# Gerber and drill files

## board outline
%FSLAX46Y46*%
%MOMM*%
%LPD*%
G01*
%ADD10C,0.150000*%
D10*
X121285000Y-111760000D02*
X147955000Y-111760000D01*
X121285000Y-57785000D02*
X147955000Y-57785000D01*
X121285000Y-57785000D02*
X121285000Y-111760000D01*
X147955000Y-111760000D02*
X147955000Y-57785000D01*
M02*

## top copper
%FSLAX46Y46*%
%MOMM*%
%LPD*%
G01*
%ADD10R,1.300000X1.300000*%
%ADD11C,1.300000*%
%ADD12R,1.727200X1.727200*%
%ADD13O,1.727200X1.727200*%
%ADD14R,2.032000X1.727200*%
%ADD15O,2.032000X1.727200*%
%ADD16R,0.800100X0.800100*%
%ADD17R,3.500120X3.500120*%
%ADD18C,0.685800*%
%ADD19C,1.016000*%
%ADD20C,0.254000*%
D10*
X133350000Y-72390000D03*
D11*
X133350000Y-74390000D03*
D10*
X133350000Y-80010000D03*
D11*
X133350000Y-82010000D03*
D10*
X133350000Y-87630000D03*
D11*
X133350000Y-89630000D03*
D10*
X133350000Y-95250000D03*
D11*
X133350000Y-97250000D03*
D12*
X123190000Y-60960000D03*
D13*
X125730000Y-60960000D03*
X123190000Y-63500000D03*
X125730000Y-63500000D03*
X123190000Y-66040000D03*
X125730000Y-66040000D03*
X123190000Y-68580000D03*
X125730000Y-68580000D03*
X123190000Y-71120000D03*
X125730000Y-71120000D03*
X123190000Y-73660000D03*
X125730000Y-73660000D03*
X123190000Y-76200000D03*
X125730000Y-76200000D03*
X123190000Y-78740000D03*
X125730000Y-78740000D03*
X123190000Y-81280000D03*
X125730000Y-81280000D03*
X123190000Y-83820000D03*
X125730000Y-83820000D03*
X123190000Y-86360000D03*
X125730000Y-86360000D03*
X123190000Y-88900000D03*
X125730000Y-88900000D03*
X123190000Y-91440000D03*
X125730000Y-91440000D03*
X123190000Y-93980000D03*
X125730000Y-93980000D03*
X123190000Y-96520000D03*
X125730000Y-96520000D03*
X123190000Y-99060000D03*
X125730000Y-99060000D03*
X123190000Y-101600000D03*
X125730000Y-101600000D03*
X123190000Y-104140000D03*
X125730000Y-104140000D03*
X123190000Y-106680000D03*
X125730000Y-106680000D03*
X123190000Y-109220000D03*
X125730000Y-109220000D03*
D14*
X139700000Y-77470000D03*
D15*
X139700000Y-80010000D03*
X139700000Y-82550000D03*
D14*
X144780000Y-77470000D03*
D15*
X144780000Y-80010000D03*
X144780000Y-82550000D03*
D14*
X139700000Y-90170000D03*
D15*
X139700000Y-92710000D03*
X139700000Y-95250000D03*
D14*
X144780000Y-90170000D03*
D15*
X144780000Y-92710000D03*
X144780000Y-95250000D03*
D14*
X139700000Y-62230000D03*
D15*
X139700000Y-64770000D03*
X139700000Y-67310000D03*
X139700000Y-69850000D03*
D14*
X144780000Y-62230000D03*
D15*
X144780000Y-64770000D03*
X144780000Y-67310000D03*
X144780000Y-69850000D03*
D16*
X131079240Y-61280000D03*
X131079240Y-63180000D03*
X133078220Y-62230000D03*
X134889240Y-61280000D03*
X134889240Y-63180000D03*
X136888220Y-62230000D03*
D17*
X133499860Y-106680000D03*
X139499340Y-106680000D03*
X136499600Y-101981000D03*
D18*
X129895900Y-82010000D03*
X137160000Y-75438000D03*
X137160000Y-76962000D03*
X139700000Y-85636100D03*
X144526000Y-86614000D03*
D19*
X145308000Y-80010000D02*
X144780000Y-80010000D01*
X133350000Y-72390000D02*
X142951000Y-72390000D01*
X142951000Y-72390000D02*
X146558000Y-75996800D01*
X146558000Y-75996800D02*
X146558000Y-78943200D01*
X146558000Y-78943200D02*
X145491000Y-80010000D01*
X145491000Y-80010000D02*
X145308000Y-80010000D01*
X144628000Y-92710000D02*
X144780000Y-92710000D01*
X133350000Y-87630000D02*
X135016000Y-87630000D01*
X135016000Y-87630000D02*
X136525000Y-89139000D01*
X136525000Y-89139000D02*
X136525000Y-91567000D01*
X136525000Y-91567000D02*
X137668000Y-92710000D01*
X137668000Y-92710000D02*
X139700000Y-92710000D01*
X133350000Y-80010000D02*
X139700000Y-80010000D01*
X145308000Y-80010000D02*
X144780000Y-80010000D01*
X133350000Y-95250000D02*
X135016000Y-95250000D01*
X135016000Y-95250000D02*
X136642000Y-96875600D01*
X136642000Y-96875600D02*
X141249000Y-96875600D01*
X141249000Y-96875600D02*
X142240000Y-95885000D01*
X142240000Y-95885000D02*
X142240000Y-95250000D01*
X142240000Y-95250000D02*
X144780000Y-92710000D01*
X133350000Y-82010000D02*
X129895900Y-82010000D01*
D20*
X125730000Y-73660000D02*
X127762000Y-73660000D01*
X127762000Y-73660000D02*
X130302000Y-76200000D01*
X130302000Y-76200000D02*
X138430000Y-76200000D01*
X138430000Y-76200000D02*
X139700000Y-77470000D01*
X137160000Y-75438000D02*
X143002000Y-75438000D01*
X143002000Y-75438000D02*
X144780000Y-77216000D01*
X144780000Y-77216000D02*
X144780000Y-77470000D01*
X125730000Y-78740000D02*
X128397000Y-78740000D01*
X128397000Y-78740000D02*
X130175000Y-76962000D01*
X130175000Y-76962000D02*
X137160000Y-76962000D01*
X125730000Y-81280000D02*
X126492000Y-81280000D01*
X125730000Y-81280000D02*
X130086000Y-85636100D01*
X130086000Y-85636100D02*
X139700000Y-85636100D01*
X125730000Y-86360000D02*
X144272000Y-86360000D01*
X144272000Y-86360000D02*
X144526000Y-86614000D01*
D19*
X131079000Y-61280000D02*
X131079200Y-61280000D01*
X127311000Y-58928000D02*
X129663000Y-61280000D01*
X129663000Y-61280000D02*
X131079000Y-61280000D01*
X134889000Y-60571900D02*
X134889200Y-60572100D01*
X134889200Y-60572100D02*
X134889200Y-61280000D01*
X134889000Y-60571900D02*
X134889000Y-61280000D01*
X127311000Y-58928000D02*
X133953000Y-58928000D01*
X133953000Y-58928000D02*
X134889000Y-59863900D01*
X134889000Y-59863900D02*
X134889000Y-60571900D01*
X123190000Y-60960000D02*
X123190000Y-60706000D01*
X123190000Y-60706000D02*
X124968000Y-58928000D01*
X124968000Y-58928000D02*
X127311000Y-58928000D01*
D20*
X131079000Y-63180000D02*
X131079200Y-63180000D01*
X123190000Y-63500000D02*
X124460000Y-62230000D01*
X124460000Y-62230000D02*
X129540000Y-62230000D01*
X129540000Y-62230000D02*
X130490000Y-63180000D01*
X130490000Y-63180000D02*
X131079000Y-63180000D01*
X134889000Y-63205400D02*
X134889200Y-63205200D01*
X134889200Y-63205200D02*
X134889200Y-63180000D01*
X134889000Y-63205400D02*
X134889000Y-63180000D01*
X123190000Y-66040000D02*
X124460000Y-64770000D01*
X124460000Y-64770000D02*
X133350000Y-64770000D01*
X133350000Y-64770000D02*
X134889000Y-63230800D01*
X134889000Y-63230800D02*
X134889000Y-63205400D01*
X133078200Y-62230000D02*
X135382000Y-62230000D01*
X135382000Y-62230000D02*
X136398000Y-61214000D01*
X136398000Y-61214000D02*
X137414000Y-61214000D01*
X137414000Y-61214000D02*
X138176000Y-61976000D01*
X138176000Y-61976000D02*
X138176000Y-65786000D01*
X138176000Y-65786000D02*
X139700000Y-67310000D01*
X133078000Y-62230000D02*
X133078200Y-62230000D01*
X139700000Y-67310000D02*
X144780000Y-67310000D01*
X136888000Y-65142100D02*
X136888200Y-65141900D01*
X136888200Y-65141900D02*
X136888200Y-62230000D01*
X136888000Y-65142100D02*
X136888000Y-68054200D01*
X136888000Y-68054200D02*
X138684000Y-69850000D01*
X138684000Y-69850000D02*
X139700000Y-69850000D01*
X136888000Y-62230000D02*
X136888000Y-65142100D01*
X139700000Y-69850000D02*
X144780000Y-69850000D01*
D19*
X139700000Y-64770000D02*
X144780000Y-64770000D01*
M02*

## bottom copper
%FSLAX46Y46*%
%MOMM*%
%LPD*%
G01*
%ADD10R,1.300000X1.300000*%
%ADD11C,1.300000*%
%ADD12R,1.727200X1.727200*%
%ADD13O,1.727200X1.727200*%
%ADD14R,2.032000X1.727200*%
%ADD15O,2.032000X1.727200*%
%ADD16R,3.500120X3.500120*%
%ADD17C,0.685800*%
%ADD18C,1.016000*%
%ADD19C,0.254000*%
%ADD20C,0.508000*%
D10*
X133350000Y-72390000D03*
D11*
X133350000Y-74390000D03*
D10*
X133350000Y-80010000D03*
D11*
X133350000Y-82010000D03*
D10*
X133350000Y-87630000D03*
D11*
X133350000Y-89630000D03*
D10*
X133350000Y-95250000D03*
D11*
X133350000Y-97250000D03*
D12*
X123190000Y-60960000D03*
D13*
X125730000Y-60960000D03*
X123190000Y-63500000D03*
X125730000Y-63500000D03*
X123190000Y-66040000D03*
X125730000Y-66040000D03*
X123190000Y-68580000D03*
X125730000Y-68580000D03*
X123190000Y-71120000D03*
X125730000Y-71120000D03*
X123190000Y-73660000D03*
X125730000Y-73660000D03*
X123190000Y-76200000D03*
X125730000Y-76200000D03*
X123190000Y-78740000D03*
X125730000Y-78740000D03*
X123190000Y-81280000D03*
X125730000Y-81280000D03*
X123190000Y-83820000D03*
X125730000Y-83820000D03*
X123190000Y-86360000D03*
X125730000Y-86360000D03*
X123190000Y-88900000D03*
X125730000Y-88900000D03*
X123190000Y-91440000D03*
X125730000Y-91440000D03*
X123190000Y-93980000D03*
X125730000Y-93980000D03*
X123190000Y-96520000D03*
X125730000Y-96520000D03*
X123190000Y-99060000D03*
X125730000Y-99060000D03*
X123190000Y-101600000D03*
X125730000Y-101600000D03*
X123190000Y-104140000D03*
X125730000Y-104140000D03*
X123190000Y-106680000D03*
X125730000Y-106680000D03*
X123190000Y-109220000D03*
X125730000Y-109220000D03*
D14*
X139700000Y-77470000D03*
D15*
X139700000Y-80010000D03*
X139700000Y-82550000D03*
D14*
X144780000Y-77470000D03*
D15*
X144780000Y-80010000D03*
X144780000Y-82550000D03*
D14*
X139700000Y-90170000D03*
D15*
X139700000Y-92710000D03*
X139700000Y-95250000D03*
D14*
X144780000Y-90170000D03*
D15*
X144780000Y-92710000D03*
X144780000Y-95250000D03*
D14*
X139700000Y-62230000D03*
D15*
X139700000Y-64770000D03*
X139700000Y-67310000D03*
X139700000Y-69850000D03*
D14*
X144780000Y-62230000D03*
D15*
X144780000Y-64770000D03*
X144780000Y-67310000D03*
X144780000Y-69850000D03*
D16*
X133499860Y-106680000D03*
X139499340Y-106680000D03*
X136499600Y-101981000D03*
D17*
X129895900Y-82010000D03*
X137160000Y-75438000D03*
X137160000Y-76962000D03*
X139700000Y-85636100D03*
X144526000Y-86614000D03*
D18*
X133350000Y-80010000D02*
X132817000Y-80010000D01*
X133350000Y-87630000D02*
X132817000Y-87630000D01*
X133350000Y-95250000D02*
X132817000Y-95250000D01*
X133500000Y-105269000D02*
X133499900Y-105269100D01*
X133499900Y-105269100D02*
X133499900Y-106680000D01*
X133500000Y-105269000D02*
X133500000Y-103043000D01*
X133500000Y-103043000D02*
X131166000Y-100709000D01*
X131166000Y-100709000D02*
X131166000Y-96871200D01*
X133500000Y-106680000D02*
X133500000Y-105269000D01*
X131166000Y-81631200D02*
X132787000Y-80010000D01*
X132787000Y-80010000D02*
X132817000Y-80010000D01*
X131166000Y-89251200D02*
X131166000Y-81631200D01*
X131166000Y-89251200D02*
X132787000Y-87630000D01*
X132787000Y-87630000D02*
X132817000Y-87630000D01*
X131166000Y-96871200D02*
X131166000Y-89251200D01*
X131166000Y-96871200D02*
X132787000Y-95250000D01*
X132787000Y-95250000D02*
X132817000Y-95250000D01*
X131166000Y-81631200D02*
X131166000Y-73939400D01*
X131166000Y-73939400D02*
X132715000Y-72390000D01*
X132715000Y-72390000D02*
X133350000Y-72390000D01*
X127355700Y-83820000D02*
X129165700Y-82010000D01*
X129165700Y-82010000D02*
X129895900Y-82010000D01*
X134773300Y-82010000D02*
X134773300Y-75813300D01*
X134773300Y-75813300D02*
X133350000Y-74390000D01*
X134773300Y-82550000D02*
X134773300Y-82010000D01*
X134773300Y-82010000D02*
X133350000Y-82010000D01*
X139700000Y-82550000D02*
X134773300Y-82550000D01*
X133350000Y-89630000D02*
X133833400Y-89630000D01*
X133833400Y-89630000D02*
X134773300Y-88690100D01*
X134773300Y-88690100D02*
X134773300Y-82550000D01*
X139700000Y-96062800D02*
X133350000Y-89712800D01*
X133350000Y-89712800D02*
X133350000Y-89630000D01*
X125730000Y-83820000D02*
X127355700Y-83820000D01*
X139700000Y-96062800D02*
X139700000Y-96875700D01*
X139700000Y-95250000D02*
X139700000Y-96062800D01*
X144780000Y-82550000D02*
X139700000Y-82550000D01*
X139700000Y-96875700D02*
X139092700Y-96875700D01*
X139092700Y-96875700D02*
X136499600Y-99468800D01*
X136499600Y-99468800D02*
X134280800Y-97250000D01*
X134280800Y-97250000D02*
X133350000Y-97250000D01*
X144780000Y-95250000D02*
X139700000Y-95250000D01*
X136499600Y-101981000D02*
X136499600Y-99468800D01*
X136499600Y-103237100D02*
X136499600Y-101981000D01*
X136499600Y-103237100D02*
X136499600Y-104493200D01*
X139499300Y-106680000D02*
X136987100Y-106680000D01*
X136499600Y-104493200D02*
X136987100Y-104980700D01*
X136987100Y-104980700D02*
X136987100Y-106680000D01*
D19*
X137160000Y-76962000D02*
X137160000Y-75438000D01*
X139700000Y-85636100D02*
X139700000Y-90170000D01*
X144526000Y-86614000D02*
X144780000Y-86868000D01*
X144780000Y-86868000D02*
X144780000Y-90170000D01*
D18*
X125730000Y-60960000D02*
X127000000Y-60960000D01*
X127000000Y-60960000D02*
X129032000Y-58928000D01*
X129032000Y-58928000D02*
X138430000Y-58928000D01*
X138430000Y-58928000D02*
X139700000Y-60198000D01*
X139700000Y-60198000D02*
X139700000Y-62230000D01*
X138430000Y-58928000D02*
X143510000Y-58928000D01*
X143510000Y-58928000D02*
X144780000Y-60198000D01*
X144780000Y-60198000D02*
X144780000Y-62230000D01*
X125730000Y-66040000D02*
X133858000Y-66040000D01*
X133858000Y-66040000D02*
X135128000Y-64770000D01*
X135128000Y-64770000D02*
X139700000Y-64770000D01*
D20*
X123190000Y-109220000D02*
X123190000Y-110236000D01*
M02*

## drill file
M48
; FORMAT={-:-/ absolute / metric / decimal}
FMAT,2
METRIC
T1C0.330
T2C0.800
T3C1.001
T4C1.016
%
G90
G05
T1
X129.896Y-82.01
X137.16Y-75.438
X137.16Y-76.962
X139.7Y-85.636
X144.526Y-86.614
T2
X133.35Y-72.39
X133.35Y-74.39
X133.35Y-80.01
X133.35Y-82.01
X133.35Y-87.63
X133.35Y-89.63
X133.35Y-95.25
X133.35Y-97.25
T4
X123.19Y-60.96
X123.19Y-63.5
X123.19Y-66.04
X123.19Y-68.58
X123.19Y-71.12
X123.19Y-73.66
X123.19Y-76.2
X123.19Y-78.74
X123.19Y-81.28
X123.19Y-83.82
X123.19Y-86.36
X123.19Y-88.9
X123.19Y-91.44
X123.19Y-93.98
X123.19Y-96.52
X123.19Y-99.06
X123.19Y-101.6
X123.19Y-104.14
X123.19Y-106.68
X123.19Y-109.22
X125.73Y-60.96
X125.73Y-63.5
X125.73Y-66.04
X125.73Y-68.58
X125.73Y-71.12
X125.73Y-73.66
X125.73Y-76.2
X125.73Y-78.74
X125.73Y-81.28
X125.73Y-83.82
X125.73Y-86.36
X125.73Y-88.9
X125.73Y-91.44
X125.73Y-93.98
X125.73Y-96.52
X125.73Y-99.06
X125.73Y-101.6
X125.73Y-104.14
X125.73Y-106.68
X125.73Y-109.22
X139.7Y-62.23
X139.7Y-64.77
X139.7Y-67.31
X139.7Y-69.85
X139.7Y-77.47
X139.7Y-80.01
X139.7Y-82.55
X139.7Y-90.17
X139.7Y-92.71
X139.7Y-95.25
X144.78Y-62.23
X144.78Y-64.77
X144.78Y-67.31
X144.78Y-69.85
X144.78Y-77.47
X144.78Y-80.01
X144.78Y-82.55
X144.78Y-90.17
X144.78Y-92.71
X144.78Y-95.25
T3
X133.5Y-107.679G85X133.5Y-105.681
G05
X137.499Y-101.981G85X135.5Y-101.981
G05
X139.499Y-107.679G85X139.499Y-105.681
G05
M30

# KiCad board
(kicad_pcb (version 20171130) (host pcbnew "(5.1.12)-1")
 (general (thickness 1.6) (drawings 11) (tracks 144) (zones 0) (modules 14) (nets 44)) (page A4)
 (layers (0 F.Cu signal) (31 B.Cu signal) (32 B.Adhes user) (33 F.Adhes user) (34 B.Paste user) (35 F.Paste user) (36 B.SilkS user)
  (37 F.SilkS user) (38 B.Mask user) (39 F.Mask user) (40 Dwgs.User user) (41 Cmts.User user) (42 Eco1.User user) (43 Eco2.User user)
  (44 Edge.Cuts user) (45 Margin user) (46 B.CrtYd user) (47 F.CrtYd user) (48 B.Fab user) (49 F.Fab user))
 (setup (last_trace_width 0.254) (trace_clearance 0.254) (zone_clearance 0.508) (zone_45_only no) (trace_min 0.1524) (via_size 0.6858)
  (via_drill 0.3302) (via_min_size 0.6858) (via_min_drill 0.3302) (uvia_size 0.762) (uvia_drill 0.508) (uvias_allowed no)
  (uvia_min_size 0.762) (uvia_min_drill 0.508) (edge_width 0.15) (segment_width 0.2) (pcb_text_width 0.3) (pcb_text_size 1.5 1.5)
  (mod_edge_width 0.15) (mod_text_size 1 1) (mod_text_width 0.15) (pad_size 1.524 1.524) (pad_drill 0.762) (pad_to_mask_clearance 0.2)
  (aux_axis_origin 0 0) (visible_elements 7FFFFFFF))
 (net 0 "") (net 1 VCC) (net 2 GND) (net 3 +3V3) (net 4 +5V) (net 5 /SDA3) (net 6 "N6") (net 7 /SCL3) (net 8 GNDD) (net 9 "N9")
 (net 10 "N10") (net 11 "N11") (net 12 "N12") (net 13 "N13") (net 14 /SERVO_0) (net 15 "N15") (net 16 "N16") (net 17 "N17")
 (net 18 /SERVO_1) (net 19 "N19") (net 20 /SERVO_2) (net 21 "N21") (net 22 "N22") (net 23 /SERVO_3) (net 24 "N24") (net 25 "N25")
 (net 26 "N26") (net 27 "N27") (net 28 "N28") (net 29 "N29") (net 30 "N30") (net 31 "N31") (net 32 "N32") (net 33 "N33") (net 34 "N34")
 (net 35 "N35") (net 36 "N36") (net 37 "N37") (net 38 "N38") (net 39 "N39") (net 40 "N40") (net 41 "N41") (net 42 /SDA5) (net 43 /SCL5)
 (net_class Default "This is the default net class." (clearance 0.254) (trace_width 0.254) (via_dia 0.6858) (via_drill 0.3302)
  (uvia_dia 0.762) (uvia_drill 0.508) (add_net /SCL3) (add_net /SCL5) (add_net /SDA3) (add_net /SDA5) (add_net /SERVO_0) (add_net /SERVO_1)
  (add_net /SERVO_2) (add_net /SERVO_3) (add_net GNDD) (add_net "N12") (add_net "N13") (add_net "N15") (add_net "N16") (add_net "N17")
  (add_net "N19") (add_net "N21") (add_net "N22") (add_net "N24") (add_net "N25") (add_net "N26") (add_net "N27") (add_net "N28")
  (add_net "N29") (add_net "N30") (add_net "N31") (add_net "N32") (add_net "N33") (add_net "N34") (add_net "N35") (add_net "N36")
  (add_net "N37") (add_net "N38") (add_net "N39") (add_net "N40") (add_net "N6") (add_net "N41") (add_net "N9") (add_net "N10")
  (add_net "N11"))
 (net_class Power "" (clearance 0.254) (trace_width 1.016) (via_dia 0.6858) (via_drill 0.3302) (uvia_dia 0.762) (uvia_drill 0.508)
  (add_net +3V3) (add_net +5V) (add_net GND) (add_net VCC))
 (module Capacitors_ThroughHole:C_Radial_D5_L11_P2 (layer F.Cu) (at 133.35 72.39 270)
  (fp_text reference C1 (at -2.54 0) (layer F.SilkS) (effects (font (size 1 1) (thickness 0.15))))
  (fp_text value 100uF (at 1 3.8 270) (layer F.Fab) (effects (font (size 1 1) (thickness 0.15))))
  (pad 1 thru_hole rect (at 0 0 270) (size 1.3 1.3) (drill 0.8) (layers *.Cu *.Mask F.SilkS) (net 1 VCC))
  (pad 2 thru_hole circle (at 2 0 270) (size 1.3 1.3) (drill 0.8) (layers *.Cu *.Mask F.SilkS) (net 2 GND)))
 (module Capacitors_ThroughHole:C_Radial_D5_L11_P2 (layer F.Cu) (at 133.35 80.01 270)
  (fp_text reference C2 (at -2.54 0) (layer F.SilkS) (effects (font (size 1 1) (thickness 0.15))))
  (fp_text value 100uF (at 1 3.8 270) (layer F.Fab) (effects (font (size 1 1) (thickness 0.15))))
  (pad 1 thru_hole rect (at 0 0 270) (size 1.3 1.3) (drill 0.8) (layers *.Cu *.Mask F.SilkS) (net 1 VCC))
  (pad 2 thru_hole circle (at 2 0 270) (size 1.3 1.3) (drill 0.8) (layers *.Cu *.Mask F.SilkS) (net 2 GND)))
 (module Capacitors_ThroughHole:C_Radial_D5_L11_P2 (layer F.Cu) (at 133.35 87.63 270)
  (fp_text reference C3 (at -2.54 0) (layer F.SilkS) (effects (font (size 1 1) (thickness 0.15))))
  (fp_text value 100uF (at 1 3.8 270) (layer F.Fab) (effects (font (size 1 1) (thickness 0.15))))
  (pad 1 thru_hole rect (at 0 0 270) (size 1.3 1.3) (drill 0.8) (layers *.Cu *.Mask F.SilkS) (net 1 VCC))
  (pad 2 thru_hole circle (at 2 0 270) (size 1.3 1.3) (drill 0.8) (layers *.Cu *.Mask F.SilkS) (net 2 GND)))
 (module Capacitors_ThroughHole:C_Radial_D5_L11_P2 (layer F.Cu) (at 133.35 95.25 270)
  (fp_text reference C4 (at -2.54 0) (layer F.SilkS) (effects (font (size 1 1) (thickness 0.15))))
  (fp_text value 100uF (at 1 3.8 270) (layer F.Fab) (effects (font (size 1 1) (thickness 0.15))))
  (pad 1 thru_hole rect (at 0 0 270) (size 1.3 1.3) (drill 0.8) (layers *.Cu *.Mask F.SilkS) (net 1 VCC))
  (pad 2 thru_hole circle (at 2 0 270) (size 1.3 1.3) (drill 0.8) (layers *.Cu *.Mask F.SilkS) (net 2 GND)))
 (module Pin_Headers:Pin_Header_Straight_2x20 (layer F.Cu) (at 123.19 60.96)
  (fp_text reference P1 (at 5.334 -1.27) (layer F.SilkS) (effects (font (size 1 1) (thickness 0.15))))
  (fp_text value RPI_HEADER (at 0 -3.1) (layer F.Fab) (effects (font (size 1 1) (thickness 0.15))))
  (pad 1 thru_hole rect (at 0 0) (size 1.7272 1.7272) (drill 1.016) (layers *.Cu *.Mask F.SilkS) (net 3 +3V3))
  (pad 2 thru_hole oval (at 2.54 0) (size 1.7272 1.7272) (drill 1.016) (layers *.Cu *.Mask F.SilkS) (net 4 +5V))
  (pad 3 thru_hole oval (at 0 2.54) (size 1.7272 1.7272) (drill 1.016) (layers *.Cu *.Mask F.SilkS) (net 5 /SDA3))
  (pad 4 thru_hole oval (at 2.54 2.54) (size 1.7272 1.7272) (drill 1.016) (layers *.Cu *.Mask F.SilkS) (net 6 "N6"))
  (pad 5 thru_hole oval (at 0 5.08) (size 1.7272 1.7272) (drill 1.016) (layers *.Cu *.Mask F.SilkS) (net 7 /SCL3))
  (pad 6 thru_hole oval (at 2.54 5.08) (size 1.7272 1.7272) (drill 1.016) (layers *.Cu *.Mask F.SilkS) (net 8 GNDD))
  (pad 7 thru_hole oval (at 0 7.62) (size 1.7272 1.7272) (drill 1.016) (layers *.Cu *.Mask F.SilkS) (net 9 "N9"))
  (pad 8 thru_hole oval (at 2.54 7.62) (size 1.7272 1.7272) (drill 1.016) (layers *.Cu *.Mask F.SilkS) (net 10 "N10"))
  (pad 9 thru_hole oval (at 0 10.16) (size 1.7272 1.7272) (drill 1.016) (layers *.Cu *.Mask F.SilkS) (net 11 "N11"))
  (pad 10 thru_hole oval (at 2.54 10.16) (size 1.7272 1.7272) (drill 1.016) (layers *.Cu *.Mask F.SilkS) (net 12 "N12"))
  (pad 11 thru_hole oval (at 0 12.7) (size 1.7272 1.7272) (drill 1.016) (layers *.Cu *.Mask F.SilkS) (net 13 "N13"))
  (pad 12 thru_hole oval (at 2.54 12.7) (size 1.7272 1.7272) (drill 1.016) (layers *.Cu *.Mask F.SilkS) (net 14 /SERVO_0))
  (pad 13 thru_hole oval (at 0 15.24) (size 1.7272 1.7272) (drill 1.016) (layers *.Cu *.Mask F.SilkS) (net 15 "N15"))
  (pad 14 thru_hole oval (at 2.54 15.24) (size 1.7272 1.7272) (drill 1.016) (layers *.Cu *.Mask F.SilkS) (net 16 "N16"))
  (pad 15 thru_hole oval (at 0 17.78) (size 1.7272 1.7272) (drill 1.016) (layers *.Cu *.Mask F.SilkS) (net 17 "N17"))
  (pad 16 thru_hole oval (at 2.54 17.78) (size 1.7272 1.7272) (drill 1.016) (layers *.Cu *.Mask F.SilkS) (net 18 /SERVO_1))
  (pad 17 thru_hole oval (at 0 20.32) (size 1.7272 1.7272) (drill 1.016) (layers *.Cu *.Mask F.SilkS) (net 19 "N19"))
  (pad 18 thru_hole oval (at 2.54 20.32) (size 1.7272 1.7272) (drill 1.016) (layers *.Cu *.Mask F.SilkS) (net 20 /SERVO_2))
  (pad 19 thru_hole oval (at 0 22.86) (size 1.7272 1.7272) (drill 1.016) (layers *.Cu *.Mask F.SilkS) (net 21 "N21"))
  (pad 20 thru_hole oval (at 2.54 22.86) (size 1.7272 1.7272) (drill 1.016) (layers *.Cu *.Mask F.SilkS) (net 2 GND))
  (pad 21 thru_hole oval (at 0 25.4) (size 1.7272 1.7272) (drill 1.016) (layers *.Cu *.Mask F.SilkS) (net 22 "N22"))
  (pad 22 thru_hole oval (at 2.54 25.4) (size 1.7272 1.7272) (drill 1.016) (layers *.Cu *.Mask F.SilkS) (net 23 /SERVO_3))
  (pad 23 thru_hole oval (at 0 27.94) (size 1.7272 1.7272) (drill 1.016) (layers *.Cu *.Mask F.SilkS) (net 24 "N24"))
  (pad 24 thru_hole oval (at 2.54 27.94) (size 1.7272 1.7272) (drill 1.016) (layers *.Cu *.Mask F.SilkS) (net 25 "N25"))
  (pad 25 thru_hole oval (at 0 30.48) (size 1.7272 1.7272) (drill 1.016) (layers *.Cu *.Mask F.SilkS) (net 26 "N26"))
  (pad 26 thru_hole oval (at 2.54 30.48) (size 1.7272 1.7272) (drill 1.016) (layers *.Cu *.Mask F.SilkS) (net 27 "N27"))
  (pad 27 thru_hole oval (at 0 33.02) (size 1.7272 1.7272) (drill 1.016) (layers *.Cu *.Mask F.SilkS) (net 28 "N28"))
  (pad 28 thru_hole oval (at 2.54 33.02) (size 1.7272 1.7272) (drill 1.016) (layers *.Cu *.Mask F.SilkS) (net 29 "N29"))
  (pad 29 thru_hole oval (at 0 35.56) (size 1.7272 1.7272) (drill 1.016) (layers *.Cu *.Mask F.SilkS) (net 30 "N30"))
  (pad 30 thru_hole oval (at 2.54 35.56) (size 1.7272 1.7272) (drill 1.016) (layers *.Cu *.Mask F.SilkS) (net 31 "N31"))
  (pad 31 thru_hole oval (at 0 38.1) (size 1.7272 1.7272) (drill 1.016) (layers *.Cu *.Mask F.SilkS) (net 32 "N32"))
  (pad 32 thru_hole oval (at 2.54 38.1) (size 1.7272 1.7272) (drill 1.016) (layers *.Cu *.Mask F.SilkS) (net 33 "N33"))
  (pad 33 thru_hole oval (at 0 40.64) (size 1.7272 1.7272) (drill 1.016) (layers *.Cu *.Mask F.SilkS) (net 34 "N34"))
  (pad 34 thru_hole oval (at 2.54 40.64) (size 1.7272 1.7272) (drill 1.016) (layers *.Cu *.Mask F.SilkS) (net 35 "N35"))
  (pad 35 thru_hole oval (at 0 43.18) (size 1.7272 1.7272) (drill 1.016) (layers *.Cu *.Mask F.SilkS) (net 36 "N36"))
  (pad 36 thru_hole oval (at 2.54 43.18) (size 1.7272 1.7272) (drill 1.016) (layers *.Cu *.Mask F.SilkS) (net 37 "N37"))
  (pad 37 thru_hole oval (at 0 45.72) (size 1.7272 1.7272) (drill 1.016) (layers *.Cu *.Mask F.SilkS) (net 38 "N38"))
  (pad 38 thru_hole oval (at 2.54 45.72) (size 1.7272 1.7272) (drill 1.016) (layers *.Cu *.Mask F.SilkS) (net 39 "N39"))
  (pad 39 thru_hole oval (at 0 48.26) (size 1.7272 1.7272) (drill 1.016) (layers *.Cu *.Mask F.SilkS) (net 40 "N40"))
  (pad 40 thru_hole oval (at 2.54 48.26) (size 1.7272 1.7272) (drill 1.016) (layers *.Cu *.Mask F.SilkS) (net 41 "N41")))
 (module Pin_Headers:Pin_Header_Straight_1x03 (layer F.Cu) (at 139.7 77.47)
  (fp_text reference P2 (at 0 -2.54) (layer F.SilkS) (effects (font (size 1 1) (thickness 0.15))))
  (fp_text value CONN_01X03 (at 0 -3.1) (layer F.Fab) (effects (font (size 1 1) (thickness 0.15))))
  (pad 1 thru_hole rect (at 0 0) (size 2.032 1.7272) (drill 1.016) (layers *.Cu *.Mask F.SilkS) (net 14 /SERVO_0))
  (pad 2 thru_hole oval (at 0 2.54) (size 2.032 1.7272) (drill 1.016) (layers *.Cu *.Mask F.SilkS) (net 1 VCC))
  (pad 3 thru_hole oval (at 0 5.08) (size 2.032 1.7272) (drill 1.016) (layers *.Cu *.Mask F.SilkS) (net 2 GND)))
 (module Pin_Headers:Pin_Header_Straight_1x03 (layer F.Cu) (at 144.78 77.47)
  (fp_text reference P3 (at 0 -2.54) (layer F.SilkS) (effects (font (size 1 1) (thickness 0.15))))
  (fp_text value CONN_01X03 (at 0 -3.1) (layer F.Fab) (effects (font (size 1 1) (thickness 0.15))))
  (pad 1 thru_hole rect (at 0 0) (size 2.032 1.7272) (drill 1.016) (layers *.Cu *.Mask F.SilkS) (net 18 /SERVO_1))
  (pad 2 thru_hole oval (at 0 2.54) (size 2.032 1.7272) (drill 1.016) (layers *.Cu *.Mask F.SilkS) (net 1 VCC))
  (pad 3 thru_hole oval (at 0 5.08) (size 2.032 1.7272) (drill 1.016) (layers *.Cu *.Mask F.SilkS) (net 2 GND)))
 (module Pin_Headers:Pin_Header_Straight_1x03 (layer F.Cu) (at 139.7 90.17)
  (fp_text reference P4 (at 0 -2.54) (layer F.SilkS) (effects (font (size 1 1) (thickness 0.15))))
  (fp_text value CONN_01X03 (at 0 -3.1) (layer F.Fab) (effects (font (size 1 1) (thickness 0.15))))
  (pad 1 thru_hole rect (at 0 0) (size 2.032 1.7272) (drill 1.016) (layers *.Cu *.Mask F.SilkS) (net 20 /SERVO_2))
  (pad 2 thru_hole oval (at 0 2.54) (size 2.032 1.7272) (drill 1.016) (layers *.Cu *.Mask F.SilkS) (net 1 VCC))
  (pad 3 thru_hole oval (at 0 5.08) (size 2.032 1.7272) (drill 1.016) (layers *.Cu *.Mask F.SilkS) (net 2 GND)))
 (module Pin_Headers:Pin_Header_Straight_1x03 (layer F.Cu) (at 144.78 90.17)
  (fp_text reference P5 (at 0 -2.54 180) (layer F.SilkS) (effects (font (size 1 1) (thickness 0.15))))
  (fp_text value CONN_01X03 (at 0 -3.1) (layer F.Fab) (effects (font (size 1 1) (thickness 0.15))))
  (pad 1 thru_hole rect (at 0 0) (size 2.032 1.7272) (drill 1.016) (layers *.Cu *.Mask F.SilkS) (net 23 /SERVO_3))
  (pad 2 thru_hole oval (at 0 2.54) (size 2.032 1.7272) (drill 1.016) (layers *.Cu *.Mask F.SilkS) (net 1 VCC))
  (pad 3 thru_hole oval (at 0 5.08) (size 2.032 1.7272) (drill 1.016) (layers *.Cu *.Mask F.SilkS) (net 2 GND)))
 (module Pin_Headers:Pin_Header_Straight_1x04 (layer F.Cu) (at 139.7 62.23)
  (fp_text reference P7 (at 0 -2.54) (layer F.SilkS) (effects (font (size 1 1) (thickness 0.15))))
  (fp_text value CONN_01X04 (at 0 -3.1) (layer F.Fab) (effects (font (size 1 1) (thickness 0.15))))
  (pad 1 thru_hole rect (at 0 0) (size 2.032 1.7272) (drill 1.016) (layers *.Cu *.Mask F.SilkS) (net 4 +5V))
  (pad 2 thru_hole oval (at 0 2.54) (size 2.032 1.7272) (drill 1.016) (layers *.Cu *.Mask F.SilkS) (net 8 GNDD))
  (pad 3 thru_hole oval (at 0 5.08) (size 2.032 1.7272) (drill 1.016) (layers *.Cu *.Mask F.SilkS) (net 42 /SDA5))
  (pad 4 thru_hole oval (at 0 7.62) (size 2.032 1.7272) (drill 1.016) (layers *.Cu *.Mask F.SilkS) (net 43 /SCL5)))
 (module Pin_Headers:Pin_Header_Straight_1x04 (layer F.Cu) (at 144.78 62.23)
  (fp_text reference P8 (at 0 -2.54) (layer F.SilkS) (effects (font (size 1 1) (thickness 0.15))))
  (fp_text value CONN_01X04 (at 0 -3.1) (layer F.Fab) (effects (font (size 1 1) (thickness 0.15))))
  (pad 1 thru_hole rect (at 0 0) (size 2.032 1.7272) (drill 1.016) (layers *.Cu *.Mask F.SilkS) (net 4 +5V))
  (pad 2 thru_hole oval (at 0 2.54) (size 2.032 1.7272) (drill 1.016) (layers *.Cu *.Mask F.SilkS) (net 8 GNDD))
  (pad 3 thru_hole oval (at 0 5.08) (size 2.032 1.7272) (drill 1.016) (layers *.Cu *.Mask F.SilkS) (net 42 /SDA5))
  (pad 4 thru_hole oval (at 0 7.62) (size 2.032 1.7272) (drill 1.016) (layers *.Cu *.Mask F.SilkS) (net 43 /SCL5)))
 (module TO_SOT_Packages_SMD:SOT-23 (layer F.Cu) (at 132.08 62.23 270)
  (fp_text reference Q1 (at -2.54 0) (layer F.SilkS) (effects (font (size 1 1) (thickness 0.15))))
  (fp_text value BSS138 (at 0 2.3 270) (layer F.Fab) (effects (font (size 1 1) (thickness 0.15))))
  (pad 1 smd rect (at -0.95 1.00076 270) (size 0.8001 0.8001) (layers F.Cu F.Paste F.Mask) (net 3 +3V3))
  (pad 2 smd rect (at 0.95 1.00076 270) (size 0.8001 0.8001) (layers F.Cu F.Paste F.Mask) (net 5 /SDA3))
  (pad 3 smd rect (at 0 -0.99822 270) (size 0.8001 0.8001) (layers F.Cu F.Paste F.Mask) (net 42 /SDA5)))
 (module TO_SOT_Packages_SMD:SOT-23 (layer F.Cu) (at 135.89 62.23 270)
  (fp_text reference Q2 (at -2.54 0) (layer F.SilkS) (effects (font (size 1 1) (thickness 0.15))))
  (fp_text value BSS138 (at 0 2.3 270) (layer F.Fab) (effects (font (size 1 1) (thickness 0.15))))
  (pad 1 smd rect (at -0.95 1.00076 270) (size 0.8001 0.8001) (layers F.Cu F.Paste F.Mask) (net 3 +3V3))
  (pad 2 smd rect (at 0.95 1.00076 270) (size 0.8001 0.8001) (layers F.Cu F.Paste F.Mask) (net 7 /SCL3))
  (pad 3 smd rect (at 0 -0.99822 270) (size 0.8001 0.8001) (layers F.Cu F.Paste F.Mask) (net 43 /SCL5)))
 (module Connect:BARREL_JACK (layer F.Cu) (at 139.7 106.68 180)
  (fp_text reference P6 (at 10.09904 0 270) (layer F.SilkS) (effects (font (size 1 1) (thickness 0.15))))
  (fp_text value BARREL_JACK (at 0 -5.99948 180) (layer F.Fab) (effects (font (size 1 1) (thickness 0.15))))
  (pad 1 thru_hole rect (at 6.20014 0 180) (size 3.50012 3.50012) (drill oval 1.00076 2.99974) (layers *.Cu *.Mask F.SilkS) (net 1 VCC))
  (pad 2 thru_hole rect (at 0.20066 0 180) (size 3.50012 3.50012) (drill oval 1.00076 2.99974) (layers *.Cu *.Mask F.SilkS) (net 2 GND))
  (pad 3 thru_hole rect (at 3.2004 4.699 180) (size 3.50012 3.50012) (drill oval 2.99974 1.00076) (layers *.Cu *.Mask F.SilkS) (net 2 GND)))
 (gr_line (start 121.285 111.76) (end 147.955 111.76) (angle 90) (layer Edge.Cuts) (width 0.15))
 (gr_line (start 121.285 57.785) (end 147.955 57.785) (angle 90) (layer Edge.Cuts) (width 0.15))
 (gr_line (start 121.285 57.785) (end 121.285 111.76) (layer Edge.Cuts) (width 0.15))
 (gr_line (start 147.955 111.76) (end 147.955 57.785) (layer Edge.Cuts) (width 0.15))
 (segment (start 133.35 80.01) (end 132.817 80.01) (width 1.016) (layer B.Cu) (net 1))
 (segment (start 133.35 87.63) (end 132.817 87.63) (width 1.016) (layer B.Cu) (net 1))
 (segment (start 133.35 95.25) (end 132.817 95.25) (width 1.016) (layer B.Cu) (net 1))
 (segment (start 133.5 105.269) (end 133.4999 105.2691) (width 1.016) (layer B.Cu) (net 1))
 (segment (start 133.4999 105.2691) (end 133.4999 106.68) (width 1.016) (layer B.Cu) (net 1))
 (segment (start 133.5 105.269) (end 133.5 103.043) (width 1.016) (layer B.Cu) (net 1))
 (segment (start 133.5 103.043) (end 131.166 100.709) (width 1.016) (layer B.Cu) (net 1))
 (segment (start 131.166 100.709) (end 131.166 96.8712) (width 1.016) (layer B.Cu) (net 1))
 (segment (start 133.5 106.68) (end 133.5 105.269) (width 1.016) (layer B.Cu) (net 1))
 (segment (start 145.308 80.01) (end 144.78 80.01) (width 1.016) (layer F.Cu) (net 1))
 (segment (start 133.35 72.39) (end 142.951 72.39) (width 1.016) (layer F.Cu) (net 1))
 (segment (start 142.951 72.39) (end 146.558 75.9968) (width 1.016) (layer F.Cu) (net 1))
 (segment (start 146.558 75.9968) (end 146.558 78.9432) (width 1.016) (layer F.Cu) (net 1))
 (segment (start 146.558 78.9432) (end 145.491 80.01) (width 1.016) (layer F.Cu) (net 1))
 (segment (start 145.491 80.01) (end 145.308 80.01) (width 1.016) (layer F.Cu) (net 1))
 (segment (start 131.166 81.6312) (end 132.787 80.01) (width 1.016) (layer B.Cu) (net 1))
 (segment (start 132.787 80.01) (end 132.817 80.01) (width 1.016) (layer B.Cu) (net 1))
 (segment (start 131.166 89.2512) (end 131.166 81.6312) (width 1.016) (layer B.Cu) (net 1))
 (segment (start 131.166 89.2512) (end 132.787 87.63) (width 1.016) (layer B.Cu) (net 1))
 (segment (start 132.787 87.63) (end 132.817 87.63) (width 1.016) (layer B.Cu) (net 1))
 (segment (start 131.166 96.8712) (end 131.166 89.2512) (width 1.016) (layer B.Cu) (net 1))
 (segment (start 131.166 96.8712) (end 132.787 95.25) (width 1.016) (layer B.Cu) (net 1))
 (segment (start 132.787 95.25) (end 132.817 95.25) (width 1.016) (layer B.Cu) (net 1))
 (segment (start 144.628 92.71) (end 144.78 92.71) (width 1.016) (layer F.Cu) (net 1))
 (segment (start 133.35 87.63) (end 135.016 87.63) (width 1.016) (layer F.Cu) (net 1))
 (segment (start 135.016 87.63) (end 136.525 89.139) (width 1.016) (layer F.Cu) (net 1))
 (segment (start 136.525 89.139) (end 136.525 91.567) (width 1.016) (layer F.Cu) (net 1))
 (segment (start 136.525 91.567) (end 137.668 92.71) (width 1.016) (layer F.Cu) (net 1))
 (segment (start 137.668 92.71) (end 139.7 92.71) (width 1.016) (layer F.Cu) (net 1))
 (segment (start 133.35 80.01) (end 139.7 80.01) (width 1.016) (layer F.Cu) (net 1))
 (segment (start 145.308 80.01) (end 144.78 80.01) (width 1.016) (layer F.Cu) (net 1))
 (segment (start 133.35 95.25) (end 135.016 95.25) (width 1.016) (layer F.Cu) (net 1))
 (segment (start 135.016 95.25) (end 136.642 96.8756) (width 1.016) (layer F.Cu) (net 1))
 (segment (start 136.642 96.8756) (end 141.249 96.8756) (width 1.016) (layer F.Cu) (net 1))
 (segment (start 141.249 96.8756) (end 142.24 95.885) (width 1.016) (layer F.Cu) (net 1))
 (segment (start 142.24 95.885) (end 142.24 95.25) (width 1.016) (layer F.Cu) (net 1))
 (segment (start 142.24 95.25) (end 144.78 92.71) (width 1.016) (layer F.Cu) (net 1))
 (segment (start 131.166 81.6312) (end 131.166 73.9394) (width 1.016) (layer B.Cu) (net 1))
 (segment (start 131.166 73.9394) (end 132.715 72.39) (width 1.016) (layer B.Cu) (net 1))
 (segment (start 132.715 72.39) (end 133.35 72.39) (width 1.016) (layer B.Cu) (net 1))
 (segment (start 133.35 82.01) (end 129.8959 82.01) (width 1.016) (layer F.Cu) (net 2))
 (segment (start 127.3557 83.82) (end 129.1657 82.01) (width 1.016) (layer B.Cu) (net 2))
 (segment (start 129.1657 82.01) (end 129.8959 82.01) (width 1.016) (layer B.Cu) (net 2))
 (segment (start 134.7733 82.01) (end 134.7733 75.8133) (width 1.016) (layer B.Cu) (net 2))
 (segment (start 134.7733 75.8133) (end 133.35 74.39) (width 1.016) (layer B.Cu) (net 2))
 (segment (start 134.7733 82.55) (end 134.7733 82.01) (width 1.016) (layer B.Cu) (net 2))
 (segment (start 134.7733 82.01) (end 133.35 82.01) (width 1.016) (layer B.Cu) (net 2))
 (segment (start 139.7 82.55) (end 134.7733 82.55) (width 1.016) (layer B.Cu) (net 2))
 (segment (start 133.35 89.63) (end 133.8334 89.63) (width 1.016) (layer B.Cu) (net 2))
 (segment (start 133.8334 89.63) (end 134.7733 88.6901) (width 1.016) (layer B.Cu) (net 2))
 (segment (start 134.7733 88.6901) (end 134.7733 82.55) (width 1.016) (layer B.Cu) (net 2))
 (segment (start 139.7 96.0628) (end 133.35 89.7128) (width 1.016) (layer B.Cu) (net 2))
 (segment (start 133.35 89.7128) (end 133.35 89.63) (width 1.016) (layer B.Cu) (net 2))
 (segment (start 125.73 83.82) (end 127.3557 83.82) (width 1.016) (layer B.Cu) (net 2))
 (segment (start 139.7 96.0628) (end 139.7 96.8757) (width 1.016) (layer B.Cu) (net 2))
 (segment (start 139.7 95.25) (end 139.7 96.0628) (width 1.016) (layer B.Cu) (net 2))
 (segment (start 144.78 82.55) (end 139.7 82.55) (width 1.016) (layer B.Cu) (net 2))
 (segment (start 139.7 96.8757) (end 139.0927 96.8757) (width 1.016) (layer B.Cu) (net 2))
 (segment (start 139.0927 96.8757) (end 136.4996 99.4688) (width 1.016) (layer B.Cu) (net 2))
 (segment (start 136.4996 99.4688) (end 134.2808 97.25) (width 1.016) (layer B.Cu) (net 2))
 (segment (start 134.2808 97.25) (end 133.35 97.25) (width 1.016) (layer B.Cu) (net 2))
 (segment (start 144.78 95.25) (end 139.7 95.25) (width 1.016) (layer B.Cu) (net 2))
 (segment (start 136.4996 101.981) (end 136.4996 99.4688) (width 1.016) (layer B.Cu) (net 2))
 (segment (start 136.4996 103.2371) (end 136.4996 101.981) (width 1.016) (layer B.Cu) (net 2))
 (segment (start 136.4996 103.2371) (end 136.4996 104.4932) (width 1.016) (layer B.Cu) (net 2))
 (segment (start 139.4993 106.68) (end 136.9871 106.68) (width 1.016) (layer B.Cu) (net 2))
 (segment (start 136.4996 104.4932) (end 136.9871 104.9807) (width 1.016) (layer B.Cu) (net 2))
 (segment (start 136.9871 104.9807) (end 136.9871 106.68) (width 1.016) (layer B.Cu) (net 2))
 (via (at 129.8959 82.01) (size 0.6858) (layers F.Cu B.Cu) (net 2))
 (segment (start 125.73 73.66) (end 127.762 73.66) (width 0.254) (layer F.Cu) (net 14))
 (segment (start 127.762 73.66) (end 130.302 76.2) (width 0.254) (layer F.Cu) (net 14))
 (segment (start 130.302 76.2) (end 138.43 76.2) (width 0.254) (layer F.Cu) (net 14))
 (segment (start 138.43 76.2) (end 139.7 77.47) (width 0.254) (layer F.Cu) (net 14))
 (segment (start 137.16 75.438) (end 143.002 75.438) (width 0.254) (layer F.Cu) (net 18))
 (segment (start 143.002 75.438) (end 144.78 77.216) (width 0.254) (layer F.Cu) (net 18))
 (segment (start 144.78 77.216) (end 144.78 77.47) (width 0.254) (layer F.Cu) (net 18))
 (segment (start 137.16 76.962) (end 137.16 75.438) (width 0.254) (layer B.Cu) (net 18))
 (segment (start 125.73 78.74) (end 128.397 78.74) (width 0.254) (layer F.Cu) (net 18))
 (segment (start 128.397 78.74) (end 130.175 76.962) (width 0.254) (layer F.Cu) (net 18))
 (segment (start 130.175 76.962) (end 137.16 76.962) (width 0.254) (layer F.Cu) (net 18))
 (via (at 137.16 75.438) (size 0.6858) (layers F.Cu B.Cu) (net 18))
 (via (at 137.16 76.962) (size 0.6858) (layers F.Cu B.Cu) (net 18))
 (segment (start 125.73 81.28) (end 126.492 81.28) (width 0.254) (layer F.Cu) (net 20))
 (segment (start 125.73 81.28) (end 130.086 85.6361) (width 0.254) (layer F.Cu) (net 20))
 (segment (start 130.086 85.6361) (end 139.7 85.6361) (width 0.254) (layer F.Cu) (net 20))
 (segment (start 139.7 85.6361) (end 139.7 90.17) (width 0.254) (layer B.Cu) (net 20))
 (via (at 139.7 85.6361) (size 0.6858) (layers F.Cu B.Cu) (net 20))
 (segment (start 125.73 86.36) (end 144.272 86.36) (width 0.254) (layer F.Cu) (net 23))
 (segment (start 144.272 86.36) (end 144.526 86.614) (width 0.254) (layer F.Cu) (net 23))
 (segment (start 144.526 86.614) (end 144.78 86.868) (width 0.254) (layer B.Cu) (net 23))
 (segment (start 144.78 86.868) (end 144.78 90.17) (width 0.254) (layer B.Cu) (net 23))
 (via (at 144.526 86.614) (size 0.6858) (layers F.Cu B.Cu) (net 23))
 (segment (start 131.079 61.28) (end 131.0792 61.28) (width 1.016) (layer F.Cu) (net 3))
 (segment (start 127.311 58.928) (end 129.663 61.28) (width 1.016) (layer F.Cu) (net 3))
 (segment (start 129.663 61.28) (end 131.079 61.28) (width 1.016) (layer F.Cu) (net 3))
 (segment (start 134.889 60.5719) (end 134.8892 60.5721) (width 1.016) (layer F.Cu) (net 3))
 (segment (start 134.8892 60.5721) (end 134.8892 61.28) (width 1.016) (layer F.Cu) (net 3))
 (segment (start 134.889 60.5719) (end 134.889 61.28) (width 1.016) (layer F.Cu) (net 3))
 (segment (start 127.311 58.928) (end 133.953 58.928) (width 1.016) (layer F.Cu) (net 3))
 (segment (start 133.953 58.928) (end 134.889 59.8639) (width 1.016) (layer F.Cu) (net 3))
 (segment (start 134.889 59.8639) (end 134.889 60.5719) (width 1.016) (layer F.Cu) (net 3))
 (segment (start 123.19 60.96) (end 123.19 60.706) (width 1.016) (layer F.Cu) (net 3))
 (segment (start 123.19 60.706) (end 124.968 58.928) (width 1.016) (layer F.Cu) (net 3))
 (segment (start 124.968 58.928) (end 127.311 58.928) (width 1.016) (layer F.Cu) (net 3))
 (segment (start 125.73 60.96) (end 127 60.96) (width 1.016) (layer B.Cu) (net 4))
 (segment (start 127 60.96) (end 129.032 58.928) (width 1.016) (layer B.Cu) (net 4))
 (segment (start 129.032 58.928) (end 138.43 58.928) (width 1.016) (layer B.Cu) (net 4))
 (segment (start 138.43 58.928) (end 139.7 60.198) (width 1.016) (layer B.Cu) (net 4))
 (segment (start 139.7 60.198) (end 139.7 62.23) (width 1.016) (layer B.Cu) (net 4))
 (segment (start 138.43 58.928) (end 143.51 58.928) (width 1.016) (layer B.Cu) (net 4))
 (segment (start 143.51 58.928) (end 144.78 60.198) (width 1.016) (layer B.Cu) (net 4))
 (segment (start 144.78 60.198) (end 144.78 62.23) (width 1.016) (layer B.Cu) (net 4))
 (segment (start 131.079 63.18) (end 131.0792 63.18) (width 0.254) (layer F.Cu) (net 5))
 (segment (start 123.19 63.5) (end 124.46 62.23) (width 0.254) (layer F.Cu) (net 5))
 (segment (start 124.46 62.23) (end 129.54 62.23) (width 0.254) (layer F.Cu) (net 5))
 (segment (start 129.54 62.23) (end 130.49 63.18) (width 0.254) (layer F.Cu) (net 5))
 (segment (start 130.49 63.18) (end 131.079 63.18) (width 0.254) (layer F.Cu) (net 5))
 (segment (start 134.889 63.2054) (end 134.8892 63.2052) (width 0.254) (layer F.Cu) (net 7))
 (segment (start 134.8892 63.2052) (end 134.8892 63.18) (width 0.254) (layer F.Cu) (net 7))
 (segment (start 134.889 63.2054) (end 134.889 63.18) (width 0.254) (layer F.Cu) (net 7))
 (segment (start 123.19 66.04) (end 124.46 64.77) (width 0.254) (layer F.Cu) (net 7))
 (segment (start 124.46 64.77) (end 133.35 64.77) (width 0.254) (layer F.Cu) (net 7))
 (segment (start 133.35 64.77) (end 134.889 63.2308) (width 0.254) (layer F.Cu) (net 7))
 (segment (start 134.889 63.2308) (end 134.889 63.2054) (width 0.254) (layer F.Cu) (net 7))
 (segment (start 133.0782 62.23) (end 135.382 62.23) (width 0.254) (layer F.Cu) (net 42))
 (segment (start 135.382 62.23) (end 136.398 61.214) (width 0.254) (layer F.Cu) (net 42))
 (segment (start 136.398 61.214) (end 137.414 61.214) (width 0.254) (layer F.Cu) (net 42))
 (segment (start 137.414 61.214) (end 138.176 61.976) (width 0.254) (layer F.Cu) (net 42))
 (segment (start 138.176 61.976) (end 138.176 65.786) (width 0.254) (layer F.Cu) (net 42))
 (segment (start 138.176 65.786) (end 139.7 67.31) (width 0.254) (layer F.Cu) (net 42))
 (segment (start 133.078 62.23) (end 133.0782 62.23) (width 0.254) (layer F.Cu) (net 42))
 (segment (start 139.7 67.31) (end 144.78 67.31) (width 0.254) (layer F.Cu) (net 42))
 (segment (start 136.888 65.1421) (end 136.8882 65.1419) (width 0.254) (layer F.Cu) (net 43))
 (segment (start 136.8882 65.1419) (end 136.8882 62.23) (width 0.254) (layer F.Cu) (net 43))
 (segment (start 136.888 65.1421) (end 136.888 68.0542) (width 0.254) (layer F.Cu) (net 43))
 (segment (start 136.888 68.0542) (end 138.684 69.85) (width 0.254) (layer F.Cu) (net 43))
 (segment (start 138.684 69.85) (end 139.7 69.85) (width 0.254) (layer F.Cu) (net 43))
 (segment (start 136.888 62.23) (end 136.888 65.1421) (width 0.254) (layer F.Cu) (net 43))
 (segment (start 139.7 69.85) (end 144.78 69.85) (width 0.254) (layer F.Cu) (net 43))
 (segment (start 139.7 64.77) (end 144.78 64.77) (width 1.016) (layer F.Cu) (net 8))
 (segment (start 125.73 66.04) (end 133.858 66.04) (width 1.016) (layer B.Cu) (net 8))
 (segment (start 133.858 66.04) (end 135.128 64.77) (width 1.016) (layer B.Cu) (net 8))
 (segment (start 135.128 64.77) (end 139.7 64.77) (width 1.016) (layer B.Cu) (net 8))
 (segment (start 123.19 109.22) (end 123.19 110.236) (width 0.508) (layer B.Cu) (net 40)))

